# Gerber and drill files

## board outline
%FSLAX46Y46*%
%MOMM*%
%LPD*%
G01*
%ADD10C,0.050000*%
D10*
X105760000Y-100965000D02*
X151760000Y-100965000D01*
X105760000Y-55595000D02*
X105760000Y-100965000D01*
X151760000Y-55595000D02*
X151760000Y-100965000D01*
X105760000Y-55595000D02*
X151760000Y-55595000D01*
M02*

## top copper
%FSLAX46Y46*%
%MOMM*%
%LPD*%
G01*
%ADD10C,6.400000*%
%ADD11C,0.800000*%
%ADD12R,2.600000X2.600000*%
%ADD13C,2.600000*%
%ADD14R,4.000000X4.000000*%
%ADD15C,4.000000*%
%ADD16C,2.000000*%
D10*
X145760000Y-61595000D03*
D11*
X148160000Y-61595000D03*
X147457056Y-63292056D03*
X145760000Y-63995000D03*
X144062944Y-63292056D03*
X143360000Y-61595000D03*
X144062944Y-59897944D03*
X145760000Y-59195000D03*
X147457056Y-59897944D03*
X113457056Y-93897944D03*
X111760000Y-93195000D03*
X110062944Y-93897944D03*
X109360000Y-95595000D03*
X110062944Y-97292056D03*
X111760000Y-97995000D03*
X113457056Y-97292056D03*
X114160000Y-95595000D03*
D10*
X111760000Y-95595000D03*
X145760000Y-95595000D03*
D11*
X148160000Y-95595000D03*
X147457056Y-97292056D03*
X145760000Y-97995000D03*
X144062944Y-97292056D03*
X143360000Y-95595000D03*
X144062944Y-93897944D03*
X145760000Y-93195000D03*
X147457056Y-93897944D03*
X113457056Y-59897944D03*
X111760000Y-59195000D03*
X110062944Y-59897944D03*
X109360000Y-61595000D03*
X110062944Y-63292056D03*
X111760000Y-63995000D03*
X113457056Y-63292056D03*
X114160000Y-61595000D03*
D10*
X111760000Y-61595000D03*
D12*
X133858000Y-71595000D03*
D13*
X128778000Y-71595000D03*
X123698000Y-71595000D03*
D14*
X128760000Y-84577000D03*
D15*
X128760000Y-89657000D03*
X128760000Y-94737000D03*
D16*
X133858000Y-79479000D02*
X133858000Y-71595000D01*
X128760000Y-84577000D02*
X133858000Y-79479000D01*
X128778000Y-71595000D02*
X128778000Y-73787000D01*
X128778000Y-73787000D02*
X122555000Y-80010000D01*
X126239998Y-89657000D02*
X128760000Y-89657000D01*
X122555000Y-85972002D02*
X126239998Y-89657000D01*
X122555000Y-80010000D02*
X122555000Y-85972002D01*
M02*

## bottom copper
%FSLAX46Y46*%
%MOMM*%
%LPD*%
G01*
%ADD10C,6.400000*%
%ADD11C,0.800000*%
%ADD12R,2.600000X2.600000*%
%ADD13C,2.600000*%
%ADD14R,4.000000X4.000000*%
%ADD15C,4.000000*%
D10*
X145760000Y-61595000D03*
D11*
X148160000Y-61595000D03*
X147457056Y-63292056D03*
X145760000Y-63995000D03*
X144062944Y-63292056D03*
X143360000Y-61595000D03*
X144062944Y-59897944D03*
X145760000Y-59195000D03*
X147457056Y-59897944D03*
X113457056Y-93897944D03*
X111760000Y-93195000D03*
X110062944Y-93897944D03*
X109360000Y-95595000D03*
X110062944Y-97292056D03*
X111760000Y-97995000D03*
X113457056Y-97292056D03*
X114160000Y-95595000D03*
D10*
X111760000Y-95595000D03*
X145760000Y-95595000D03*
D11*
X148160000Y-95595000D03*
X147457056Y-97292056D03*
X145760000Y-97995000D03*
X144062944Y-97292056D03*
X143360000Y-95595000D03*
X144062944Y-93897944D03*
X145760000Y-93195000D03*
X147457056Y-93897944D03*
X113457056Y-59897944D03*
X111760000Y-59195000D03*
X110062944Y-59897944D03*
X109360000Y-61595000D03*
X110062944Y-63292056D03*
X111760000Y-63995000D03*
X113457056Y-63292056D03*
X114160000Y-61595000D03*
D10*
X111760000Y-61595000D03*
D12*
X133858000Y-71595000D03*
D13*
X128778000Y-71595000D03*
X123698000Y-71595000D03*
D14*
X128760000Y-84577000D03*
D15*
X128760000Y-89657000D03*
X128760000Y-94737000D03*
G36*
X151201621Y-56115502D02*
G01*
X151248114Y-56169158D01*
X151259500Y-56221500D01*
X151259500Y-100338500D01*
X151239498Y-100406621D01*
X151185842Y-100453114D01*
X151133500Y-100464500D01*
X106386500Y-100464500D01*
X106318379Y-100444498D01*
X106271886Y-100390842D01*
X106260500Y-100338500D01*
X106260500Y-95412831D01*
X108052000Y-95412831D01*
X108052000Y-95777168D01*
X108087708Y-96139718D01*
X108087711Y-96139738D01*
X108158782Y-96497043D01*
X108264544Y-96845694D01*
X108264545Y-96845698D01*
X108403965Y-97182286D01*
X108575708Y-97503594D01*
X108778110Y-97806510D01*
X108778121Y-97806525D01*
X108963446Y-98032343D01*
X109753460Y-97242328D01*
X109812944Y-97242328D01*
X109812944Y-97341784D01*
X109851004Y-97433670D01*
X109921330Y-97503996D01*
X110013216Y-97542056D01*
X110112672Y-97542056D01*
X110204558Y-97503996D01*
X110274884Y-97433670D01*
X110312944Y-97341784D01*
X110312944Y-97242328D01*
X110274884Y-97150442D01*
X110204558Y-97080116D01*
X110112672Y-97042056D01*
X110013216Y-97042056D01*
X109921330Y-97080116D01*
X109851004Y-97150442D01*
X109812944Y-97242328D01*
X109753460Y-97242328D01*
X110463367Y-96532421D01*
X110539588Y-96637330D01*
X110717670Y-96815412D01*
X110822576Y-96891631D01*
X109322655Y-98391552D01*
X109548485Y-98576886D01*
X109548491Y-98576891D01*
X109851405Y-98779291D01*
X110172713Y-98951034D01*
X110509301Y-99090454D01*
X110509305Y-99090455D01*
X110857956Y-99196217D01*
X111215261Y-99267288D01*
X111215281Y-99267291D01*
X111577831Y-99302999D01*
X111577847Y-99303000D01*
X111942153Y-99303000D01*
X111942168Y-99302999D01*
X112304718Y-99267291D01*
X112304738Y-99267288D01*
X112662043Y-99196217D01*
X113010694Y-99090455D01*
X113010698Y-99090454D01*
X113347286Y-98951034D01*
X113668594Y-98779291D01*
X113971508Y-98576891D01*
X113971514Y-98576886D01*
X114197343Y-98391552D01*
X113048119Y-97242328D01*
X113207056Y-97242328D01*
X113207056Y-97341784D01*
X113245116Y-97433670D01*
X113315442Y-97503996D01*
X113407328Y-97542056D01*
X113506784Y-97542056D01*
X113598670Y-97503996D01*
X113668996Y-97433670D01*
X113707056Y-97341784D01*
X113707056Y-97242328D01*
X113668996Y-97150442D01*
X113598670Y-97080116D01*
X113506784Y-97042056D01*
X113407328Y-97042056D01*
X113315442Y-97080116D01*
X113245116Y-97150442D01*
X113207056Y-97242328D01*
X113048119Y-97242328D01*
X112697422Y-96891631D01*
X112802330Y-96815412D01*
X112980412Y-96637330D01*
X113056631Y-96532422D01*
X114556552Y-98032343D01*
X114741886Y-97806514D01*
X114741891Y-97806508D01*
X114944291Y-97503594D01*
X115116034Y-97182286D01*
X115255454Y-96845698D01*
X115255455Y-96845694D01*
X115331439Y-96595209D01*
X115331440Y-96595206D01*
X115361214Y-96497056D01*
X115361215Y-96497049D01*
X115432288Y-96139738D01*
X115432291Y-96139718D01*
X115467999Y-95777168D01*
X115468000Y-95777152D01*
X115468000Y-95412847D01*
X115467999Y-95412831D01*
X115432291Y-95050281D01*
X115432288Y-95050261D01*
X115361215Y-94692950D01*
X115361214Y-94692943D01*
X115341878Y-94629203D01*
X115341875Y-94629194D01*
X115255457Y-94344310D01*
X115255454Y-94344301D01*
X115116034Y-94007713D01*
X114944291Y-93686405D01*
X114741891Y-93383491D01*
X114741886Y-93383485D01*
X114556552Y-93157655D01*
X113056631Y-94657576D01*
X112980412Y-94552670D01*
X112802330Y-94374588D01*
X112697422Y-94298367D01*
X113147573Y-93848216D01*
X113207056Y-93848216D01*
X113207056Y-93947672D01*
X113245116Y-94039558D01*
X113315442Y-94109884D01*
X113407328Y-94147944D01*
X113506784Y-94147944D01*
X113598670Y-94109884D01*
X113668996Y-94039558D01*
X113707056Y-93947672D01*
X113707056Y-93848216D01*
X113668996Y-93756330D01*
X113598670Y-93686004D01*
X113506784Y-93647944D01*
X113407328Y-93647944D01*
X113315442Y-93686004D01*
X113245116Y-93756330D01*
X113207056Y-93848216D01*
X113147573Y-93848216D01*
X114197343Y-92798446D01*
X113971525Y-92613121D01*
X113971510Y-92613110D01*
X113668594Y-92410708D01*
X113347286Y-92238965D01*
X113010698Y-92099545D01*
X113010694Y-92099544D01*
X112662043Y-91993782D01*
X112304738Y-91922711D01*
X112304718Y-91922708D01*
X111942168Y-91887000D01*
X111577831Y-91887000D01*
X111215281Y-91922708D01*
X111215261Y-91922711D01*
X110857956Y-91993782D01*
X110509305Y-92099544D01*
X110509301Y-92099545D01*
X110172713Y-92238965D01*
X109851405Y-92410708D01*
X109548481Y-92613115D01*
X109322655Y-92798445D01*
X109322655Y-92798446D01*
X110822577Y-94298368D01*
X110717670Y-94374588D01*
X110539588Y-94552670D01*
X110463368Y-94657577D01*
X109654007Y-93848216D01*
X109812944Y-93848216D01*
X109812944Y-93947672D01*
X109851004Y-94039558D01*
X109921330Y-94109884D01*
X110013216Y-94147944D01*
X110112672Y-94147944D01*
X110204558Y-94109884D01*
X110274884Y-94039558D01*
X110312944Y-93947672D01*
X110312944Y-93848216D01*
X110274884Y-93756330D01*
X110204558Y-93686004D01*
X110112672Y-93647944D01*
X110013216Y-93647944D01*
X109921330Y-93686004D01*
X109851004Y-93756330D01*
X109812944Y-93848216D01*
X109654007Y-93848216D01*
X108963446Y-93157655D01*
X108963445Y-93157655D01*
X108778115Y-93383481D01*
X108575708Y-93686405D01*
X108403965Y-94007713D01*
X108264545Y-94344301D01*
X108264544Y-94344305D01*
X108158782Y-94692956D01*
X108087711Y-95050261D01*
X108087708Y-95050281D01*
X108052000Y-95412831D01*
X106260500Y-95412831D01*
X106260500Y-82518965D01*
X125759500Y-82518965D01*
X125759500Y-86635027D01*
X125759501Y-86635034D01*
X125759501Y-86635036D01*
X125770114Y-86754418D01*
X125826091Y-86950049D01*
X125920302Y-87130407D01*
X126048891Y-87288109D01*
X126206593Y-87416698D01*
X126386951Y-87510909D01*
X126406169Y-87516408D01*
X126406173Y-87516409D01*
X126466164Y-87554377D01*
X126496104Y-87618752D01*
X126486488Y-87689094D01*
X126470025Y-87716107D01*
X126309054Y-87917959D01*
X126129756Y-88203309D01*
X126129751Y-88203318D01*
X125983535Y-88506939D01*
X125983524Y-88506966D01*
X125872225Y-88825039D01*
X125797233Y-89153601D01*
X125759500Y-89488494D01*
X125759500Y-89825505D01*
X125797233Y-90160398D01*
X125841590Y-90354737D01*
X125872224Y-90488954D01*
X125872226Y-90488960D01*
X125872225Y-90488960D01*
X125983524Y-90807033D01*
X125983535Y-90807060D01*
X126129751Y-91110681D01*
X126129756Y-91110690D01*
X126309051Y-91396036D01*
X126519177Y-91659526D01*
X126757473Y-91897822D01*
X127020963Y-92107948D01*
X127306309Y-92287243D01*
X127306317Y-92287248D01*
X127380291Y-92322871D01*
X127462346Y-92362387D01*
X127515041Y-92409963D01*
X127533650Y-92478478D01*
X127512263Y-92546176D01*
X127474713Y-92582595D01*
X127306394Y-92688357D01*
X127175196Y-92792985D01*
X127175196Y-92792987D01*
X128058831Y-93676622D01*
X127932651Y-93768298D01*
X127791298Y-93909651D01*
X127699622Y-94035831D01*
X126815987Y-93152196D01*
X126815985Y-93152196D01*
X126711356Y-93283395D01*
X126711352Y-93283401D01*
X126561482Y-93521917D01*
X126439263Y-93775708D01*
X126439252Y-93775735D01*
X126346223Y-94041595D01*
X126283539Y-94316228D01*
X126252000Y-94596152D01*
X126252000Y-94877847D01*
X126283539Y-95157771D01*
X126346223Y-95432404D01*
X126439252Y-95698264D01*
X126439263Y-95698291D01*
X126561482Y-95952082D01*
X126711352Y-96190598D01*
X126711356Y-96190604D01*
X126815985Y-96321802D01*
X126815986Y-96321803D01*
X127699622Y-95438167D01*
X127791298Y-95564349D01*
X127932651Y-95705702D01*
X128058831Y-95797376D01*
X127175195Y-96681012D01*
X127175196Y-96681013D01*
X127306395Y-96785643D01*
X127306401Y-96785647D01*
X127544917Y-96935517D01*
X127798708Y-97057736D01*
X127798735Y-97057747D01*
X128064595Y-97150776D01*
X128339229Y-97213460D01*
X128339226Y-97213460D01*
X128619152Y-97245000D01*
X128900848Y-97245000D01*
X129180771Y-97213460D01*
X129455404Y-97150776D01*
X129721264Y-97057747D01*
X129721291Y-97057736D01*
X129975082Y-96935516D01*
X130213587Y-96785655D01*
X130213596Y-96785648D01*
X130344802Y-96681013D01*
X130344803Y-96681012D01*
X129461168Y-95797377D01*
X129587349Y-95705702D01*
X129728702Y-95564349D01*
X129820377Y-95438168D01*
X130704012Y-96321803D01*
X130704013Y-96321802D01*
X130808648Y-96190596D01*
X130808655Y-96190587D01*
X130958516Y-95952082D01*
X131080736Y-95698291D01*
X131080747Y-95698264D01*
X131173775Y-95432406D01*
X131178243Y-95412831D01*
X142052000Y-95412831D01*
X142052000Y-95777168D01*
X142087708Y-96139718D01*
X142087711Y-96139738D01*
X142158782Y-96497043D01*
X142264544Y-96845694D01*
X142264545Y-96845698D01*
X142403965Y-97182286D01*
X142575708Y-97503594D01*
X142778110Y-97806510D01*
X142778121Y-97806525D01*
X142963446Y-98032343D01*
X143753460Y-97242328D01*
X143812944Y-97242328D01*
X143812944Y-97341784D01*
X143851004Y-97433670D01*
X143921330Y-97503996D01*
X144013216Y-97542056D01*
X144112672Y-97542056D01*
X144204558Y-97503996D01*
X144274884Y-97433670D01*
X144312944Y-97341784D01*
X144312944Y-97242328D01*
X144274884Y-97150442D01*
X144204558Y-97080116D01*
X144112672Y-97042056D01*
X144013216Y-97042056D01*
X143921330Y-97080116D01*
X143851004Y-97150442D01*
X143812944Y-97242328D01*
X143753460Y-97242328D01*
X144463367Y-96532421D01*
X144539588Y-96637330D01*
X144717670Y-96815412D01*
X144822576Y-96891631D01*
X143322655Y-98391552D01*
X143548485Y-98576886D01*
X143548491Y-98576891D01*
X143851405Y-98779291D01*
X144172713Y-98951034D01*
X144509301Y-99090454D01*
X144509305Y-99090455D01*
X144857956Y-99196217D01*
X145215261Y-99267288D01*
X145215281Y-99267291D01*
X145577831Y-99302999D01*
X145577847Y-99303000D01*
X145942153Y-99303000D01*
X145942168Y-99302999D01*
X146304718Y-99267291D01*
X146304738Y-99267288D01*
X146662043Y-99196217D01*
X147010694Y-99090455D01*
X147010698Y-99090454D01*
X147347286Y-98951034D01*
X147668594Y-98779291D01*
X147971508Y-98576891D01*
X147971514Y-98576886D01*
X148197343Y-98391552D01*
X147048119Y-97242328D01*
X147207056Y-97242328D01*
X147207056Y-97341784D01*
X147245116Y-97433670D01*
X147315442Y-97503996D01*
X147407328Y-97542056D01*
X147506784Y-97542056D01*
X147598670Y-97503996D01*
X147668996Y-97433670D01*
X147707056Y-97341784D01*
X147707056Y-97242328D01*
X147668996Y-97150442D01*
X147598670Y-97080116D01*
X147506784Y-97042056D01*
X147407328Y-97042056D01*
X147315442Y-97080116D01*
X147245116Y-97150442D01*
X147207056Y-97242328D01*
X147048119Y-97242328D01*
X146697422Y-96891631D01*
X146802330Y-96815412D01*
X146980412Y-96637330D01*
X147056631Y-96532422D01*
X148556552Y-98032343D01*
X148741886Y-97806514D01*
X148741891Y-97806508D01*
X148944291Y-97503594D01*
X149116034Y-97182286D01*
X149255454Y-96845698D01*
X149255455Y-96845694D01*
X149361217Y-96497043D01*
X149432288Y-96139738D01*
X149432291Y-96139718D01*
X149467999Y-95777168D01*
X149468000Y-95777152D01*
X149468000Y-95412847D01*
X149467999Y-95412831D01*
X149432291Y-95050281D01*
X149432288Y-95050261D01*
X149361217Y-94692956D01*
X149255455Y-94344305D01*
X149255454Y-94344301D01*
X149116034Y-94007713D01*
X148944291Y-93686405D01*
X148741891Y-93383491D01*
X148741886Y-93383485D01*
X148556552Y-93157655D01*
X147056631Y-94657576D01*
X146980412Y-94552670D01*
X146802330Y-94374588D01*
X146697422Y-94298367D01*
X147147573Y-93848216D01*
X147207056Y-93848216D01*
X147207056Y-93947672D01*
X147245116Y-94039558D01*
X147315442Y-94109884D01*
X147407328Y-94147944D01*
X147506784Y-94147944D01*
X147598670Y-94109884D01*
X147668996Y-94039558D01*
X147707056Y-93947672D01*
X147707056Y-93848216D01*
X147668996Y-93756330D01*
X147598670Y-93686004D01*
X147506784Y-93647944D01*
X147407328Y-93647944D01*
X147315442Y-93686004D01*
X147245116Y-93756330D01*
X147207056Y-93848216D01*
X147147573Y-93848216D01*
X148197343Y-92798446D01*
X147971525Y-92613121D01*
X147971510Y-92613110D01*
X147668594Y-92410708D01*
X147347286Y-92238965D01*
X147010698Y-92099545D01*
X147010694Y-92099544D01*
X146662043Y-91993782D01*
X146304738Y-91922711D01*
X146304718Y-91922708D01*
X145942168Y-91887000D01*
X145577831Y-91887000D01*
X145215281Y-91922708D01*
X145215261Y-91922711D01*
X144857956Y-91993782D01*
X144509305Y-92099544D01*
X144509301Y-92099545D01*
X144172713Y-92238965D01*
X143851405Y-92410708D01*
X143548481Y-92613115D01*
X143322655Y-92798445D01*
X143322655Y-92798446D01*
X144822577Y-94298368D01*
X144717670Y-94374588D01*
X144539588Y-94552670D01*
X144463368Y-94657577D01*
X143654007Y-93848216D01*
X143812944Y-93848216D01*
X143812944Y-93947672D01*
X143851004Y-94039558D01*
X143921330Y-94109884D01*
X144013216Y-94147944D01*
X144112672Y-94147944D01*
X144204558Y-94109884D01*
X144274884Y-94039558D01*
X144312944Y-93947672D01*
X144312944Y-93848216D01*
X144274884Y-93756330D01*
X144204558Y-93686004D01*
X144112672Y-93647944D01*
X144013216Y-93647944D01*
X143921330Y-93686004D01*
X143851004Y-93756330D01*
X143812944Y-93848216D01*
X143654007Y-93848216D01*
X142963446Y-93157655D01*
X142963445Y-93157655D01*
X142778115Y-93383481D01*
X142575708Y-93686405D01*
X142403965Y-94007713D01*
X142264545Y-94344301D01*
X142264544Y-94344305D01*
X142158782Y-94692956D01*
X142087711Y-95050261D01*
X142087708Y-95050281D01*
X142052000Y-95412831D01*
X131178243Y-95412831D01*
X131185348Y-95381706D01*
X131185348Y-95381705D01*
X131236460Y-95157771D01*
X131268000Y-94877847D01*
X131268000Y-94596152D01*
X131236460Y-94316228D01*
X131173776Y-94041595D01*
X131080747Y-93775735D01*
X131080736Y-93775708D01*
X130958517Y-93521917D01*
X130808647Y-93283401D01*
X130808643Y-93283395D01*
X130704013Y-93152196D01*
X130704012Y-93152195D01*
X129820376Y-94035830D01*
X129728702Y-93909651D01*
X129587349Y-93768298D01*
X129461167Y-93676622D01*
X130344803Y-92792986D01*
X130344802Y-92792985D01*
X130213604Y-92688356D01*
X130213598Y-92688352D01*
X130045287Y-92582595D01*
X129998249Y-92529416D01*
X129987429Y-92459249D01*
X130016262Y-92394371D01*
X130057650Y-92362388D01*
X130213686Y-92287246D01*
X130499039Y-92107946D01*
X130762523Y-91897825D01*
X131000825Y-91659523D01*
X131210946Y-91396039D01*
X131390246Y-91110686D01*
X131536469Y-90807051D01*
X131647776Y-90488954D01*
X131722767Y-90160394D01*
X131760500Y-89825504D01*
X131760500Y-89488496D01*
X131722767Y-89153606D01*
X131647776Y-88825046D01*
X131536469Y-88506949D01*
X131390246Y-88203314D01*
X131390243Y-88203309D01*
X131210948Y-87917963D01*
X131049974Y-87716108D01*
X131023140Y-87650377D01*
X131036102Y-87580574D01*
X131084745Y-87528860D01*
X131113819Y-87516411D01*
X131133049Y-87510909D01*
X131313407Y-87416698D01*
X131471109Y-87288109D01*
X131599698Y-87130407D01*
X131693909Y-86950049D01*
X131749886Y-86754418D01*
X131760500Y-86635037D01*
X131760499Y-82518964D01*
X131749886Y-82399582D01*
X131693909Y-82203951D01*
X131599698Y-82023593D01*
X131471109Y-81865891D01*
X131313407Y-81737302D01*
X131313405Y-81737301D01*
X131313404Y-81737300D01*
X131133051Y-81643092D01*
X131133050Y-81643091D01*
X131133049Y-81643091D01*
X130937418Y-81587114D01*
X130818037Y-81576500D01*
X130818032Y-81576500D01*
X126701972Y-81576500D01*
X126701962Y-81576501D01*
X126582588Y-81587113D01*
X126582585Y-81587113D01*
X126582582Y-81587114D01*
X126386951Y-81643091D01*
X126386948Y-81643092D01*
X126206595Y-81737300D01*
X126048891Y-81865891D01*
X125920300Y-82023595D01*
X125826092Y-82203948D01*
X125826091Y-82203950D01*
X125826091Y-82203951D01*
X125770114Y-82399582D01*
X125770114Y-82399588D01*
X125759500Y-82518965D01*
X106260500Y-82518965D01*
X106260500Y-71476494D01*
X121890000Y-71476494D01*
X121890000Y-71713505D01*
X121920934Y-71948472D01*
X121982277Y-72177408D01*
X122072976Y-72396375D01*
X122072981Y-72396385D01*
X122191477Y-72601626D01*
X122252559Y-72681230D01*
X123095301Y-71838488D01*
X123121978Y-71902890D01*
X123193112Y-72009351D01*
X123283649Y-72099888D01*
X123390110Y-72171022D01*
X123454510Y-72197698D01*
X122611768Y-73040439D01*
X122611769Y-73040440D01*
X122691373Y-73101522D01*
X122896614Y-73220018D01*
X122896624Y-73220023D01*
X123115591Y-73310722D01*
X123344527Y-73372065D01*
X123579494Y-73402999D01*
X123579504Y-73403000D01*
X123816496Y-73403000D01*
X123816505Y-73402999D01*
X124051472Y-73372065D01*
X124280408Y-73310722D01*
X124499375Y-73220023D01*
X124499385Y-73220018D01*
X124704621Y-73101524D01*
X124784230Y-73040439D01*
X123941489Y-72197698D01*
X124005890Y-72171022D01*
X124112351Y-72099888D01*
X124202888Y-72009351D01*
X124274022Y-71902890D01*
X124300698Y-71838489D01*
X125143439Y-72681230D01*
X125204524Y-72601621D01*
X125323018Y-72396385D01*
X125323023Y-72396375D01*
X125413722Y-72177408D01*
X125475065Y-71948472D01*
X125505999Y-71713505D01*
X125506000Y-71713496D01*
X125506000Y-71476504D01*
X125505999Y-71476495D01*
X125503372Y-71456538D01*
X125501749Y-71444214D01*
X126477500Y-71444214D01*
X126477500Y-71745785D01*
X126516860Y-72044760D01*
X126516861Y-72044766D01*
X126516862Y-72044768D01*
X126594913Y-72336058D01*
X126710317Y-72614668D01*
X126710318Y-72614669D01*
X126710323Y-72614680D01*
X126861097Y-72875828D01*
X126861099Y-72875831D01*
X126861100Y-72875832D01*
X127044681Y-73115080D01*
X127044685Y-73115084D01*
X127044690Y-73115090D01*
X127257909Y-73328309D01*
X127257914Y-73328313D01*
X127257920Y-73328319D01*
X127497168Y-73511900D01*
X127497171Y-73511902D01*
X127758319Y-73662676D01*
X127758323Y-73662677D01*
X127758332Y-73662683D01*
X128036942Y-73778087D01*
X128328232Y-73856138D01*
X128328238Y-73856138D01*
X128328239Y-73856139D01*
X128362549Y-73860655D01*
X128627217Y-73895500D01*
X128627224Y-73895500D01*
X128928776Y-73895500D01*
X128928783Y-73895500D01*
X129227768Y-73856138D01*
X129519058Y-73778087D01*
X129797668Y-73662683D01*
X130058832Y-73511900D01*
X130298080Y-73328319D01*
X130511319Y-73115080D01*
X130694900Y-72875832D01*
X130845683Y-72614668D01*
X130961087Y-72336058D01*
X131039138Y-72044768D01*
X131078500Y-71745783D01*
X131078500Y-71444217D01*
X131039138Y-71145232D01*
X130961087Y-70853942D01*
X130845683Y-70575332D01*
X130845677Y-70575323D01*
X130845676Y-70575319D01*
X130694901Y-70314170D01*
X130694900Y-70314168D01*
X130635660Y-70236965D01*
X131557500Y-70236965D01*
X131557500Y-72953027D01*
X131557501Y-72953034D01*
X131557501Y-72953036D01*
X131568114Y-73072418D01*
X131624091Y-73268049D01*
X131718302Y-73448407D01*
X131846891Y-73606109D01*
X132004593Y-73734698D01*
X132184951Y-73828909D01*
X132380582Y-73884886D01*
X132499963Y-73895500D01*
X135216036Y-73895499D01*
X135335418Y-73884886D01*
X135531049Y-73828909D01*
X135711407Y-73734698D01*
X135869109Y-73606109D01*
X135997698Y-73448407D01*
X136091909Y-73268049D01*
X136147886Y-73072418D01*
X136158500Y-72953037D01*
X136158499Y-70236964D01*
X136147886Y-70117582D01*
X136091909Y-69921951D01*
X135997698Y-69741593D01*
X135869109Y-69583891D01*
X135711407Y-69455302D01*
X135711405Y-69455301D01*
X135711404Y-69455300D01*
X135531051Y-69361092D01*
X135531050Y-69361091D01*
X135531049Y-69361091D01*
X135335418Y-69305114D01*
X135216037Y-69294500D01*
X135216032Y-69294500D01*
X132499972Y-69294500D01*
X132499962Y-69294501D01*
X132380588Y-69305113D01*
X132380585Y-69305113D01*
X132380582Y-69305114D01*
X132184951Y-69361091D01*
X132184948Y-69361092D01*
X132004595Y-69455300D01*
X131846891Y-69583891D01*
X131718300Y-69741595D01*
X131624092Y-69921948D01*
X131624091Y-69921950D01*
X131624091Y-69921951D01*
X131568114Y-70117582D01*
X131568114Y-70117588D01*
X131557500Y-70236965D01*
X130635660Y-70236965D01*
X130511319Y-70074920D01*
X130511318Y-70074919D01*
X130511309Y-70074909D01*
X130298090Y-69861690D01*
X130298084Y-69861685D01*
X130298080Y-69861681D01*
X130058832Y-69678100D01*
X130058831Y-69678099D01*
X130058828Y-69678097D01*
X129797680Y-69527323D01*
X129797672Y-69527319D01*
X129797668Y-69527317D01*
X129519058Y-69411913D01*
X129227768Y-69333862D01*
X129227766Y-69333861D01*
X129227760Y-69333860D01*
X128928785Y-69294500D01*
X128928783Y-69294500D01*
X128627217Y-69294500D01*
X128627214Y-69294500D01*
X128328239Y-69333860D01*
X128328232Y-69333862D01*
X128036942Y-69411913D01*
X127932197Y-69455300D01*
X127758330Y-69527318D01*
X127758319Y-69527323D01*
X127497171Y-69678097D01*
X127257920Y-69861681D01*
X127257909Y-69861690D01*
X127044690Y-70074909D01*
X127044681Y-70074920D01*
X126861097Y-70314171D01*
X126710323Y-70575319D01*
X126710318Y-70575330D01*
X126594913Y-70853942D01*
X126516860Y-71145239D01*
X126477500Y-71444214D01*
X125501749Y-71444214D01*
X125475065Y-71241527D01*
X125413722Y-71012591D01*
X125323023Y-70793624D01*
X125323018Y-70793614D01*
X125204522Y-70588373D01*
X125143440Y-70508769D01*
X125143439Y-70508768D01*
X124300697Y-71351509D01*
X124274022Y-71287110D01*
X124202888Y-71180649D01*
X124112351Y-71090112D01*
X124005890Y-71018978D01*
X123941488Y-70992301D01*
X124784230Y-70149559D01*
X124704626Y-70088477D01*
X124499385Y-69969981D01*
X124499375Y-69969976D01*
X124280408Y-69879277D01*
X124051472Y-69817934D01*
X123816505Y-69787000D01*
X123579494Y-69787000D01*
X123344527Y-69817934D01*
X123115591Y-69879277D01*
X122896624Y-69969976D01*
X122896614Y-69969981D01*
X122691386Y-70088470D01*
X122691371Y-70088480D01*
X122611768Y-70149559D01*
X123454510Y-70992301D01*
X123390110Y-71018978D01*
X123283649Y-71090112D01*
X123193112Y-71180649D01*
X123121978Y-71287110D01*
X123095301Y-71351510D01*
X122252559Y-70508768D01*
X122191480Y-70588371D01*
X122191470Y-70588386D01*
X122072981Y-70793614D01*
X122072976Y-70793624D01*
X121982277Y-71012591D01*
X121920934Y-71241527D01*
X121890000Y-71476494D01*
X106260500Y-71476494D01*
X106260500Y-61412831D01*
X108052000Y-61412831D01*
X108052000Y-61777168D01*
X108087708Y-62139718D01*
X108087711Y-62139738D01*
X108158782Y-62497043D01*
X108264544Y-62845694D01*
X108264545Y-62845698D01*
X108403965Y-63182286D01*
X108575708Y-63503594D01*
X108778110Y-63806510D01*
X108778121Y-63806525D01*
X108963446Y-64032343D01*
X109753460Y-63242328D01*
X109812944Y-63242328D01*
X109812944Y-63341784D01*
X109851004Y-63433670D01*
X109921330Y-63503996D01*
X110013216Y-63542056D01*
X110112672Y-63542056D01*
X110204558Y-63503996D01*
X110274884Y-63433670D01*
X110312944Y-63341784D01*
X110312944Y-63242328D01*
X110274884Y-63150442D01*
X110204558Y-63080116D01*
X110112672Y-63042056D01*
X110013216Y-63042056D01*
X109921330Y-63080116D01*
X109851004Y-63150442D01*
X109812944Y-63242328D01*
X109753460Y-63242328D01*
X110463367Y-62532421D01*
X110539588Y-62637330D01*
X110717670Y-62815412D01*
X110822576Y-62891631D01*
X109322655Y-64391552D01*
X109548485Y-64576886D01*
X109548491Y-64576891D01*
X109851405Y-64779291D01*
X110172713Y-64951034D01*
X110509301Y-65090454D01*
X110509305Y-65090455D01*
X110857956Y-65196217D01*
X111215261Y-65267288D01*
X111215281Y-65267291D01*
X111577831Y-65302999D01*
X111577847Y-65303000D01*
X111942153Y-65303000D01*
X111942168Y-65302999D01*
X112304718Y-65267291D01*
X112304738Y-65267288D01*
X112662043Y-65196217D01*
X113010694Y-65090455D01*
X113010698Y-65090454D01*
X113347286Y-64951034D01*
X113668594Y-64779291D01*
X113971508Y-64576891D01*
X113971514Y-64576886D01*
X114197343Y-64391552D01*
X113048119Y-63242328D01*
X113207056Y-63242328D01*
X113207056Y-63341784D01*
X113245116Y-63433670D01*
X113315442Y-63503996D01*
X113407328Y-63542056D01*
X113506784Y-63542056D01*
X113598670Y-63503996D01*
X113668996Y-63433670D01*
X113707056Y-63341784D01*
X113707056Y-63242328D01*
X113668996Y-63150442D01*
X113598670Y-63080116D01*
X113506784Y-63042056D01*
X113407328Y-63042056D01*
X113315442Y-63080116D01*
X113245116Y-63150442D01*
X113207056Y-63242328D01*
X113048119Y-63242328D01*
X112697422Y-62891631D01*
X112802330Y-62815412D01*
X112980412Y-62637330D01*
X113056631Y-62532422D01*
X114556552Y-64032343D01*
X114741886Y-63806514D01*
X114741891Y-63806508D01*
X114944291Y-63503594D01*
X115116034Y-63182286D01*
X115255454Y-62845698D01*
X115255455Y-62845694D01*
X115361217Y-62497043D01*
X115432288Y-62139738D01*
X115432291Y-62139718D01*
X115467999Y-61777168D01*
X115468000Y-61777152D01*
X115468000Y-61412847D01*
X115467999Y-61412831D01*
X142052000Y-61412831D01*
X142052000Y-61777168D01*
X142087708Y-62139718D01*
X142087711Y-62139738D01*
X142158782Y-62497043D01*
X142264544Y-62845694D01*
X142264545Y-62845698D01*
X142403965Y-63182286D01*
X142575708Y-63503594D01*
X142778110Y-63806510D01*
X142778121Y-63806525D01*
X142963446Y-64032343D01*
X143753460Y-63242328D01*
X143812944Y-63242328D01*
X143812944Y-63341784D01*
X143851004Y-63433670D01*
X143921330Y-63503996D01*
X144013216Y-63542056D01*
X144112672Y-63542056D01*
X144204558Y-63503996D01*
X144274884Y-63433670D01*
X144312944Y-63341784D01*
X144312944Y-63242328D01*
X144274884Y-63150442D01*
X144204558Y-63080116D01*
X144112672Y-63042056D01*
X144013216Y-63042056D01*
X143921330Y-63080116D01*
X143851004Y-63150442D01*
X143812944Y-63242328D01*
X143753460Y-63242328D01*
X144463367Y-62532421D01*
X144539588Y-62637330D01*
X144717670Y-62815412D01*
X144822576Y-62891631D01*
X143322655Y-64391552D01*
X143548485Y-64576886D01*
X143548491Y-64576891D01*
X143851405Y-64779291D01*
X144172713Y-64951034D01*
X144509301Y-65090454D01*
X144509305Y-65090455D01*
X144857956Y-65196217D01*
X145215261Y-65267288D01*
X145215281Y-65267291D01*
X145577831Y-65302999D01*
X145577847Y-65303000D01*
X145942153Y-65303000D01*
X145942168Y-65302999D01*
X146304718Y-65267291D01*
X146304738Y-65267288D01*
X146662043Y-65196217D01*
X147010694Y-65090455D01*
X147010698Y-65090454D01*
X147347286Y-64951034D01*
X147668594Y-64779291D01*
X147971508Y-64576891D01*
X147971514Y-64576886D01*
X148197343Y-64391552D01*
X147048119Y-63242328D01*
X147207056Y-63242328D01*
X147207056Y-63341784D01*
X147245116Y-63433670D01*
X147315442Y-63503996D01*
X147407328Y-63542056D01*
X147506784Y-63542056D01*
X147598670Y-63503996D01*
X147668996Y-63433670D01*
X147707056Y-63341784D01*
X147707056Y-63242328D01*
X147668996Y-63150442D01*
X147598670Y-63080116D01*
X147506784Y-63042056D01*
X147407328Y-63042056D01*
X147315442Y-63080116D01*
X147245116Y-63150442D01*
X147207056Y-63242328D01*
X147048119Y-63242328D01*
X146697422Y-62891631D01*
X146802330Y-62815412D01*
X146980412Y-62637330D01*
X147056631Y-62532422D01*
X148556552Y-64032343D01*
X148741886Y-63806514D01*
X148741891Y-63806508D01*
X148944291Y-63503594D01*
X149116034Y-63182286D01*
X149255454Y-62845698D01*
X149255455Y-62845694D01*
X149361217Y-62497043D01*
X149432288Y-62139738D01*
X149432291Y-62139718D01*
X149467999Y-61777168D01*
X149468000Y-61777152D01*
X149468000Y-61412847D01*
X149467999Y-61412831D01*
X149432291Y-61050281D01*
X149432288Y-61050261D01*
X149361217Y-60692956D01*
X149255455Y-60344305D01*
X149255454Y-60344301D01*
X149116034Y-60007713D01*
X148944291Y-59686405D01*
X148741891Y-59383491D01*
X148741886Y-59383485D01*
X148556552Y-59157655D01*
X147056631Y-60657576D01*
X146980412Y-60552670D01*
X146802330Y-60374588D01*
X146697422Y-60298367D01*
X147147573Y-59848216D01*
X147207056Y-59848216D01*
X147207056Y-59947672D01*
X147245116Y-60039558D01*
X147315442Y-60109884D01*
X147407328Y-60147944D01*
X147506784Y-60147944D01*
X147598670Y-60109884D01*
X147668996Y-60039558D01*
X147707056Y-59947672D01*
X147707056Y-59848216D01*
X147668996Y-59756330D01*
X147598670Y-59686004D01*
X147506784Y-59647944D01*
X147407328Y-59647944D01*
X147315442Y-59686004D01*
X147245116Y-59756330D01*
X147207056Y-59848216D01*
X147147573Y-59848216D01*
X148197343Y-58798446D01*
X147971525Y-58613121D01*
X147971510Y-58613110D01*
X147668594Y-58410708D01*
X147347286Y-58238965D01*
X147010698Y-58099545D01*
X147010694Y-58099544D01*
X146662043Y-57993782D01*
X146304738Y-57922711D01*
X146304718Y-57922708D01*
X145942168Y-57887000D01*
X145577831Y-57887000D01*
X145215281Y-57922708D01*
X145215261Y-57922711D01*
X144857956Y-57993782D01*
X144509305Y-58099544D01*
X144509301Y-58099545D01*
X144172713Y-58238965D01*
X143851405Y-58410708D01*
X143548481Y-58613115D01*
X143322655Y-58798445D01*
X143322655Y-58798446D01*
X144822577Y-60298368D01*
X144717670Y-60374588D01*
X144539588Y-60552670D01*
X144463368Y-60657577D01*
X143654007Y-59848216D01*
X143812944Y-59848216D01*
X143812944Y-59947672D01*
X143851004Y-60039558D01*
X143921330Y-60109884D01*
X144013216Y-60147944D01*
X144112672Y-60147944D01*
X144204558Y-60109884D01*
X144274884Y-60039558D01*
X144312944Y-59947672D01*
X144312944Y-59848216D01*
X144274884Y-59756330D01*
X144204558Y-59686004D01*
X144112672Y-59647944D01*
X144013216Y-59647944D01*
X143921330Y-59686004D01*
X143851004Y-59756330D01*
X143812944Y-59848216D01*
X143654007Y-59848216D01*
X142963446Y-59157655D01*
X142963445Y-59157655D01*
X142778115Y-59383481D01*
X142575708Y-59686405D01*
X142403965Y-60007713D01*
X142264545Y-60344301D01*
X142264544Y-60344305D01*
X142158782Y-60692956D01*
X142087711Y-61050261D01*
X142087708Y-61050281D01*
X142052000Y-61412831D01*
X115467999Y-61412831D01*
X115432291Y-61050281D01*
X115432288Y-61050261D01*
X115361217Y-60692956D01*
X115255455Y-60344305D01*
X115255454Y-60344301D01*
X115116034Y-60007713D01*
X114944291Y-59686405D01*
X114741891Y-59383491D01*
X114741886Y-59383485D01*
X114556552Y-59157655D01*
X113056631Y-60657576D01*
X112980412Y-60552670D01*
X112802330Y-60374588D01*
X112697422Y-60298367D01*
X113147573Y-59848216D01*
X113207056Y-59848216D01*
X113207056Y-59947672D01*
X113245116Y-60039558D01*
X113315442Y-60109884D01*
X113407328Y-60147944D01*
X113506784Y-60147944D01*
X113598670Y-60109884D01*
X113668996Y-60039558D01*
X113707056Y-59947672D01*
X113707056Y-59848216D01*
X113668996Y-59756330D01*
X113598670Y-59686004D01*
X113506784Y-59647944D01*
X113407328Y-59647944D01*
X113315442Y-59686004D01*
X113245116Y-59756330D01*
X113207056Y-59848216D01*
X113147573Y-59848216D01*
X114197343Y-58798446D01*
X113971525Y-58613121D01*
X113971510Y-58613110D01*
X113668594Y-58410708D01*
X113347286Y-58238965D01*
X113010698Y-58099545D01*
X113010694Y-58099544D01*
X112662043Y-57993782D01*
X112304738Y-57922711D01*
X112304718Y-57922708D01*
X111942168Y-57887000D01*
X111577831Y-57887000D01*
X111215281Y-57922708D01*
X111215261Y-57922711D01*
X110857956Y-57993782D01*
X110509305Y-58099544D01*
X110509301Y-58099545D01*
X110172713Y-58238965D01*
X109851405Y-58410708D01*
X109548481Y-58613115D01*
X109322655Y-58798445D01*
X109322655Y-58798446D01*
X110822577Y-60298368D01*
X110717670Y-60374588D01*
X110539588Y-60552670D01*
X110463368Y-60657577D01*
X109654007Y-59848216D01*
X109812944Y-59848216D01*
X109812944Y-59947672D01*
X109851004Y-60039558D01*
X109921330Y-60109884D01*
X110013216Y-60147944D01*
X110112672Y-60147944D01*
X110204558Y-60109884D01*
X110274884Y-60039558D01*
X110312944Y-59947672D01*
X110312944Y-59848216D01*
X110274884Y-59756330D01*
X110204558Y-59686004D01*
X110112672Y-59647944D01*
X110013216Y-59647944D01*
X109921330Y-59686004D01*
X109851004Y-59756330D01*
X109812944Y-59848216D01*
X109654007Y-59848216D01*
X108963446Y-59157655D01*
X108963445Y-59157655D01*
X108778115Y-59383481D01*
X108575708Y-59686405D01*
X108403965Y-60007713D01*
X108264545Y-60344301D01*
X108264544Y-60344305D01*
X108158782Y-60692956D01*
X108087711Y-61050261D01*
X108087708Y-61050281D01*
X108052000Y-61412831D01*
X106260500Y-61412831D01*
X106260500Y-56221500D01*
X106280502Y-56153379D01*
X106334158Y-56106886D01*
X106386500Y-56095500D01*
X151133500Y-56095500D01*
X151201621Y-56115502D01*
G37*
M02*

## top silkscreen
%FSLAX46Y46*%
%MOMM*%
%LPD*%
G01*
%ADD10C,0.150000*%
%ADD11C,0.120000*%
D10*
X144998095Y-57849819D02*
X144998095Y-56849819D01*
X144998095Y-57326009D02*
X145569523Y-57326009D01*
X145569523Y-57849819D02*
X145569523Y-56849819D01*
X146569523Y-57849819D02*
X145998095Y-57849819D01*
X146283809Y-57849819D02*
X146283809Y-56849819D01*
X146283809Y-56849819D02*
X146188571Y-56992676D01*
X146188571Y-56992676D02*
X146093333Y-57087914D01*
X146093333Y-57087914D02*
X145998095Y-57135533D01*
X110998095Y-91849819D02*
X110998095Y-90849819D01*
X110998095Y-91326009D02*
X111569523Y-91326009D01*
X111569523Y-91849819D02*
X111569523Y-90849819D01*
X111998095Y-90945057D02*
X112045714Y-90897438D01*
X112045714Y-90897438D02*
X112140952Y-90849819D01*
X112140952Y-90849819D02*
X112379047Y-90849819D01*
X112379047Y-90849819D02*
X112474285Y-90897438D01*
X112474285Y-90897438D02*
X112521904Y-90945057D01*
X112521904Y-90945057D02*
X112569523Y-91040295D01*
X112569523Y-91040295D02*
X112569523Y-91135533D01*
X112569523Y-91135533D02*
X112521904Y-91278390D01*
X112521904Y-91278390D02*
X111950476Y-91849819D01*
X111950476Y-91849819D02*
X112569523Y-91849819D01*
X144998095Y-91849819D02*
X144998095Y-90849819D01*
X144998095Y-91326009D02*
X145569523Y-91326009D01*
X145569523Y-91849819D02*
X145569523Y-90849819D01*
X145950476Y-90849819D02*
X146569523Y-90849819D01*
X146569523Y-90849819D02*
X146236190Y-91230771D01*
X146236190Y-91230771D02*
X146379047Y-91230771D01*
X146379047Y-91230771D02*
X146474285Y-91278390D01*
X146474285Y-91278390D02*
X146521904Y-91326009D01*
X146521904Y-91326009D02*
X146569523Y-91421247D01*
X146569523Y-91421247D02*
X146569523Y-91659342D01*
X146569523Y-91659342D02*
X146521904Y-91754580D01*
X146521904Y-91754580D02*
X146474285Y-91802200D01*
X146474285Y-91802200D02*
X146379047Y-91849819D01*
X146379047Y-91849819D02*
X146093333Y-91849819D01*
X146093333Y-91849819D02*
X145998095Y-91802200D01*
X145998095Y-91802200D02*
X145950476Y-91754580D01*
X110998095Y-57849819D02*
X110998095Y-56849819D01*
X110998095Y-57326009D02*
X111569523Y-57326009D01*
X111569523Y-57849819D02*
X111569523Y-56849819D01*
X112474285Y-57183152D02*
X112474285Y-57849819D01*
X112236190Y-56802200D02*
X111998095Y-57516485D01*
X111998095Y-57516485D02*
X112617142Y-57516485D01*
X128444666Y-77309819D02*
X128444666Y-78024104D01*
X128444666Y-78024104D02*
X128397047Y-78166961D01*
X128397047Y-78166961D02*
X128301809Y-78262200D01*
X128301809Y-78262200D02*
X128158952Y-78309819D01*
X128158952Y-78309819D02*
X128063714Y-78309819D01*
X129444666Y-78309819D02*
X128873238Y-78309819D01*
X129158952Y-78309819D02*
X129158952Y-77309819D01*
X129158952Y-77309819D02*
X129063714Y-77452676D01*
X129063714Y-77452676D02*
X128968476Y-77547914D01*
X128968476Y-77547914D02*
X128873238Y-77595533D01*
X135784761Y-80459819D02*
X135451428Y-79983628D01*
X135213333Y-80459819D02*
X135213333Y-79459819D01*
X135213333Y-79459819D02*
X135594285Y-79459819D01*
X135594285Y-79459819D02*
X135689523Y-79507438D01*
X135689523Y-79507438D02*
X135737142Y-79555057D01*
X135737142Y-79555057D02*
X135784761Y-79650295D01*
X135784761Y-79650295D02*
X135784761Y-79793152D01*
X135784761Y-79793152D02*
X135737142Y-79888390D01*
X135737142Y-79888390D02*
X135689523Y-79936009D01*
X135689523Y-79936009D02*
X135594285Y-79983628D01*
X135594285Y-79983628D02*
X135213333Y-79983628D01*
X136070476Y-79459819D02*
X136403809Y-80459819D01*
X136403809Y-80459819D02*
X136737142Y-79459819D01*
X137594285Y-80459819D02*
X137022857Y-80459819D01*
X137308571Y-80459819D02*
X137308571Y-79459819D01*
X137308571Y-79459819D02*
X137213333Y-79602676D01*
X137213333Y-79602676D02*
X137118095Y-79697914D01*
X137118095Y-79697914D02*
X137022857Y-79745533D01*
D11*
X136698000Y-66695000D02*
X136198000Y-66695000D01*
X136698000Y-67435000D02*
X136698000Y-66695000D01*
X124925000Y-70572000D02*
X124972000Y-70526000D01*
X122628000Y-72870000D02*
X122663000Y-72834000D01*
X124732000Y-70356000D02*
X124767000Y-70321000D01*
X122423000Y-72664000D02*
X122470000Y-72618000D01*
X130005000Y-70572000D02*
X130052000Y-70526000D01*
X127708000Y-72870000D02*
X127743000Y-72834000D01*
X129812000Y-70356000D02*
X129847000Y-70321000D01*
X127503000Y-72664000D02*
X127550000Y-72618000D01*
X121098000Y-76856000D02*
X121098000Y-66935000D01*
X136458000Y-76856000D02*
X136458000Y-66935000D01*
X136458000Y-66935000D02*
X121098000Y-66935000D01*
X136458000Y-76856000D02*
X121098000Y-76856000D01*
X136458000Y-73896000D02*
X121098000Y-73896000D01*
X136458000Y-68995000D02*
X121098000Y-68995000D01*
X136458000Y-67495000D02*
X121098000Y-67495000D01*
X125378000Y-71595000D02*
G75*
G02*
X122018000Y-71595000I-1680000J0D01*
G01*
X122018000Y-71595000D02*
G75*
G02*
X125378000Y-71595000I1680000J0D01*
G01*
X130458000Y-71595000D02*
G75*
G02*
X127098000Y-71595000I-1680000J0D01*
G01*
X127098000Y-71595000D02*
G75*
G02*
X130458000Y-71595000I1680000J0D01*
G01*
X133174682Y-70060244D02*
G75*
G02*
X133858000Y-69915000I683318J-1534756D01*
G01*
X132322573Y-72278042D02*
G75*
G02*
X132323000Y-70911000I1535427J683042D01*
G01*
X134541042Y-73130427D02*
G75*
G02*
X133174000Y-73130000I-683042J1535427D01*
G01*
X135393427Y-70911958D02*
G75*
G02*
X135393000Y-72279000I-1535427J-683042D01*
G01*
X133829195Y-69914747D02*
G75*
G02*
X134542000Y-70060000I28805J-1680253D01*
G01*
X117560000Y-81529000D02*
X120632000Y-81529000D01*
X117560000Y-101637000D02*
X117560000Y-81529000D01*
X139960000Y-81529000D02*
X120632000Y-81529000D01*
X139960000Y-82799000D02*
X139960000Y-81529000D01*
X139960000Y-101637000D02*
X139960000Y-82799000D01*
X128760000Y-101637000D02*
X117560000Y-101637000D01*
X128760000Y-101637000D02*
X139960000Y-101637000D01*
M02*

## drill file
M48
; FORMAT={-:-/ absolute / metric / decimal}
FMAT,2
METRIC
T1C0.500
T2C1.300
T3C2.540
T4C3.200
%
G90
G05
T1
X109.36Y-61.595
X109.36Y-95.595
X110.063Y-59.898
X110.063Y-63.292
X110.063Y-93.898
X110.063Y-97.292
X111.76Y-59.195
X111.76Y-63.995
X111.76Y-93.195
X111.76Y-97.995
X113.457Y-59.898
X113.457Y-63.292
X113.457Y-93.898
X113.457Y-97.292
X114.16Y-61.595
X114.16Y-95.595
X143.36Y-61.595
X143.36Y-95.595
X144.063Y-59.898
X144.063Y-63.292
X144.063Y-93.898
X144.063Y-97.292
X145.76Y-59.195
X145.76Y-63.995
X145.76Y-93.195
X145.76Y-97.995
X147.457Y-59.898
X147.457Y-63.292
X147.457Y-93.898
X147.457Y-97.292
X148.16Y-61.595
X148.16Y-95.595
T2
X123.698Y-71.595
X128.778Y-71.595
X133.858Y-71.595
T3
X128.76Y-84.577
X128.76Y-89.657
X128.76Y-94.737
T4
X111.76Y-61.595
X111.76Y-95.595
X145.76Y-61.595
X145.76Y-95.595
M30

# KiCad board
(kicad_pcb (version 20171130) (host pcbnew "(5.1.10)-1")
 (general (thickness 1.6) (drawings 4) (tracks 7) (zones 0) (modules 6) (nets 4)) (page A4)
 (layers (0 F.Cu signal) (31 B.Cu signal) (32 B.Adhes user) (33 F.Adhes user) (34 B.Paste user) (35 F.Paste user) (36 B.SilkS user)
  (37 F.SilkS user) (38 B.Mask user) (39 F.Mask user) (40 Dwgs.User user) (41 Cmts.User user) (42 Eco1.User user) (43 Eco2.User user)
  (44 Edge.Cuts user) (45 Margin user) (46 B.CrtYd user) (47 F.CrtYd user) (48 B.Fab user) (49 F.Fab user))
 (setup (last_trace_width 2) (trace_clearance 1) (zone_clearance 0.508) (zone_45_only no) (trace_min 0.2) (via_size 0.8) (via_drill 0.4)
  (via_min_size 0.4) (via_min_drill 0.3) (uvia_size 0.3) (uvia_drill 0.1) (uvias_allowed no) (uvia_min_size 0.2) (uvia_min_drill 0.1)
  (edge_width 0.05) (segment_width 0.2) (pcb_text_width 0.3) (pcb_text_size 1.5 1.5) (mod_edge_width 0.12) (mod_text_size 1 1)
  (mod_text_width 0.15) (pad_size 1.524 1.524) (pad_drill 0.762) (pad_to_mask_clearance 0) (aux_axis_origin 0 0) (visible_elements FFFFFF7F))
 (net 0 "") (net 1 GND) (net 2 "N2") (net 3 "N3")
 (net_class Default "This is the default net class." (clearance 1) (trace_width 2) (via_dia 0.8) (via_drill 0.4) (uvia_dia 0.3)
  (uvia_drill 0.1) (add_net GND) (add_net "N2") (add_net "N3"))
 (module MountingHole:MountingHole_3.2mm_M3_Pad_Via (layer F.Cu) (at 145.76 61.595)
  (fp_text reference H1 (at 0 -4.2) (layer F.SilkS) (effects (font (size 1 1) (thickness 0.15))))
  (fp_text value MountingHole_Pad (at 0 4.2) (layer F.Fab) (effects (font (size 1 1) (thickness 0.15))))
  (pad 1 thru_hole circle (at 0 0) (size 6.4 6.4) (drill 3.2) (layers *.Cu *.Mask) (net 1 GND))
  (pad 1 thru_hole circle (at 2.4 0) (size 0.8 0.8) (drill 0.5) (layers *.Cu *.Mask) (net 1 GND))
  (pad 1 thru_hole circle (at 1.697056 1.697056) (size 0.8 0.8) (drill 0.5) (layers *.Cu *.Mask) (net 1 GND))
  (pad 1 thru_hole circle (at 0 2.4) (size 0.8 0.8) (drill 0.5) (layers *.Cu *.Mask) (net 1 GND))
  (pad 1 thru_hole circle (at -1.697056 1.697056) (size 0.8 0.8) (drill 0.5) (layers *.Cu *.Mask) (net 1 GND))
  (pad 1 thru_hole circle (at -2.4 0) (size 0.8 0.8) (drill 0.5) (layers *.Cu *.Mask) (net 1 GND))
  (pad 1 thru_hole circle (at -1.697056 -1.697056) (size 0.8 0.8) (drill 0.5) (layers *.Cu *.Mask) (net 1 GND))
  (pad 1 thru_hole circle (at 0 -2.4) (size 0.8 0.8) (drill 0.5) (layers *.Cu *.Mask) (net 1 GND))
  (pad 1 thru_hole circle (at 1.697056 -1.697056) (size 0.8 0.8) (drill 0.5) (layers *.Cu *.Mask) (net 1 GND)))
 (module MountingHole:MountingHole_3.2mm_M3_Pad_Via (layer F.Cu) (at 111.76 95.595)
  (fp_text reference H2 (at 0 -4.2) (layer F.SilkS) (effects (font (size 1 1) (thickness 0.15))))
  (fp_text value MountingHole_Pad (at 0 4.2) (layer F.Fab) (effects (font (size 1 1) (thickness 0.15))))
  (pad 1 thru_hole circle (at 1.697056 -1.697056) (size 0.8 0.8) (drill 0.5) (layers *.Cu *.Mask) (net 1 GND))
  (pad 1 thru_hole circle (at 0 -2.4) (size 0.8 0.8) (drill 0.5) (layers *.Cu *.Mask) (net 1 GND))
  (pad 1 thru_hole circle (at -1.697056 -1.697056) (size 0.8 0.8) (drill 0.5) (layers *.Cu *.Mask) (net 1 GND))
  (pad 1 thru_hole circle (at -2.4 0) (size 0.8 0.8) (drill 0.5) (layers *.Cu *.Mask) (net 1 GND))
  (pad 1 thru_hole circle (at -1.697056 1.697056) (size 0.8 0.8) (drill 0.5) (layers *.Cu *.Mask) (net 1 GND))
  (pad 1 thru_hole circle (at 0 2.4) (size 0.8 0.8) (drill 0.5) (layers *.Cu *.Mask) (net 1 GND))
  (pad 1 thru_hole circle (at 1.697056 1.697056) (size 0.8 0.8) (drill 0.5) (layers *.Cu *.Mask) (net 1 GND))
  (pad 1 thru_hole circle (at 2.4 0) (size 0.8 0.8) (drill 0.5) (layers *.Cu *.Mask) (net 1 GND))
  (pad 1 thru_hole circle (at 0 0) (size 6.4 6.4) (drill 3.2) (layers *.Cu *.Mask) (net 1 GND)))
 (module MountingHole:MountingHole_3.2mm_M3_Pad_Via (layer F.Cu) (at 145.76 95.595)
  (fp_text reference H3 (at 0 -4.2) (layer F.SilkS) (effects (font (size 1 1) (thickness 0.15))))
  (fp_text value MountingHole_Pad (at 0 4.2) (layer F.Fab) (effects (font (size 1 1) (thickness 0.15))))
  (pad 1 thru_hole circle (at 0 0) (size 6.4 6.4) (drill 3.2) (layers *.Cu *.Mask) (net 1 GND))
  (pad 1 thru_hole circle (at 2.4 0) (size 0.8 0.8) (drill 0.5) (layers *.Cu *.Mask) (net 1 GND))
  (pad 1 thru_hole circle (at 1.697056 1.697056) (size 0.8 0.8) (drill 0.5) (layers *.Cu *.Mask) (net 1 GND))
  (pad 1 thru_hole circle (at 0 2.4) (size 0.8 0.8) (drill 0.5) (layers *.Cu *.Mask) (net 1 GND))
  (pad 1 thru_hole circle (at -1.697056 1.697056) (size 0.8 0.8) (drill 0.5) (layers *.Cu *.Mask) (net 1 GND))
  (pad 1 thru_hole circle (at -2.4 0) (size 0.8 0.8) (drill 0.5) (layers *.Cu *.Mask) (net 1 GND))
  (pad 1 thru_hole circle (at -1.697056 -1.697056) (size 0.8 0.8) (drill 0.5) (layers *.Cu *.Mask) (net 1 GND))
  (pad 1 thru_hole circle (at 0 -2.4) (size 0.8 0.8) (drill 0.5) (layers *.Cu *.Mask) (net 1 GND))
  (pad 1 thru_hole circle (at 1.697056 -1.697056) (size 0.8 0.8) (drill 0.5) (layers *.Cu *.Mask) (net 1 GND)))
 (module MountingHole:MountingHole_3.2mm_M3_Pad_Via (layer F.Cu) (at 111.76 61.595)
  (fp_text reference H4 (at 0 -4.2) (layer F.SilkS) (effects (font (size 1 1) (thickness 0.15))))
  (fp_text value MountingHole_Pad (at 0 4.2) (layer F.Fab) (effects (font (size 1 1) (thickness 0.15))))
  (pad 1 thru_hole circle (at 1.697056 -1.697056) (size 0.8 0.8) (drill 0.5) (layers *.Cu *.Mask) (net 1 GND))
  (pad 1 thru_hole circle (at 0 -2.4) (size 0.8 0.8) (drill 0.5) (layers *.Cu *.Mask) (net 1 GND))
  (pad 1 thru_hole circle (at -1.697056 -1.697056) (size 0.8 0.8) (drill 0.5) (layers *.Cu *.Mask) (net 1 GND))
  (pad 1 thru_hole circle (at -2.4 0) (size 0.8 0.8) (drill 0.5) (layers *.Cu *.Mask) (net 1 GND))
  (pad 1 thru_hole circle (at -1.697056 1.697056) (size 0.8 0.8) (drill 0.5) (layers *.Cu *.Mask) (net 1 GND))
  (pad 1 thru_hole circle (at 0 2.4) (size 0.8 0.8) (drill 0.5) (layers *.Cu *.Mask) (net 1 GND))
  (pad 1 thru_hole circle (at 1.697056 1.697056) (size 0.8 0.8) (drill 0.5) (layers *.Cu *.Mask) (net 1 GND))
  (pad 1 thru_hole circle (at 2.4 0) (size 0.8 0.8) (drill 0.5) (layers *.Cu *.Mask) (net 1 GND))
  (pad 1 thru_hole circle (at 0 0) (size 6.4 6.4) (drill 3.2) (layers *.Cu *.Mask) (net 1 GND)))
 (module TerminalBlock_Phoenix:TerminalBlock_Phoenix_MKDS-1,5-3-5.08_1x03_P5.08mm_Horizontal (layer F.Cu) (at 133.858 71.595 180)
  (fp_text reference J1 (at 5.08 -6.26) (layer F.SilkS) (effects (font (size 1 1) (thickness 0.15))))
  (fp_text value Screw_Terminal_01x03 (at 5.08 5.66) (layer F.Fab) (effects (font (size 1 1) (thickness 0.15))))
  (fp_line (start -2.84 4.9) (end -2.34 4.9) (layer F.SilkS) (width 0.12))
  (fp_line (start -2.84 4.16) (end -2.84 4.9) (layer F.SilkS) (width 0.12))
  (fp_line (start 8.933 1.023) (end 8.886 1.069) (layer F.SilkS) (width 0.12))
  (fp_line (start 11.23 -1.275) (end 11.195 -1.239) (layer F.SilkS) (width 0.12))
  (fp_line (start 9.126 1.239) (end 9.091 1.274) (layer F.SilkS) (width 0.12))
  (fp_line (start 11.435 -1.069) (end 11.388 -1.023) (layer F.SilkS) (width 0.12))
  (fp_line (start 3.853 1.023) (end 3.806 1.069) (layer F.SilkS) (width 0.12))
  (fp_line (start 6.15 -1.275) (end 6.115 -1.239) (layer F.SilkS) (width 0.12))
  (fp_line (start 4.046 1.239) (end 4.011 1.274) (layer F.SilkS) (width 0.12))
  (fp_line (start 6.355 -1.069) (end 6.308 -1.023) (layer F.SilkS) (width 0.12))
  (fp_line (start 12.76 -5.261) (end 12.76 4.66) (layer F.SilkS) (width 0.12))
  (fp_line (start -2.6 -5.261) (end -2.6 4.66) (layer F.SilkS) (width 0.12))
  (fp_line (start -2.6 4.66) (end 12.76 4.66) (layer F.SilkS) (width 0.12))
  (fp_line (start -2.6 -5.261) (end 12.76 -5.261) (layer F.SilkS) (width 0.12))
  (fp_line (start -2.6 -2.301) (end 12.76 -2.301) (layer F.SilkS) (width 0.12))
  (fp_line (start -2.6 2.6) (end 12.76 2.6) (layer F.SilkS) (width 0.12))
  (fp_line (start -2.6 4.1) (end 12.76 4.1) (layer F.SilkS) (width 0.12))
  (fp_circle (center 10.16 0) (end 11.84 0) (layer F.SilkS) (width 0.12))
  (fp_circle (center 5.08 0) (end 6.76 0) (layer F.SilkS) (width 0.12))
  (fp_arc (start 0 0) (end 0 1.68) (angle -24) (layer F.SilkS) (width 0.12))
  (fp_arc (start 0 0) (end 1.535 0.684) (angle -48) (layer F.SilkS) (width 0.12))
  (fp_arc (start 0 0) (end 0.684 -1.535) (angle -48) (layer F.SilkS) (width 0.12))
  (fp_arc (start 0 0) (end -1.535 -0.684) (angle -48) (layer F.SilkS) (width 0.12))
  (fp_arc (start 0 0) (end -0.684 1.535) (angle -25) (layer F.SilkS) (width 0.12))
  (pad 1 thru_hole rect (at 0 0 180) (size 2.6 2.6) (drill 1.3) (layers *.Cu *.Mask) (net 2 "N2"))
  (pad 2 thru_hole circle (at 5.08 0 180) (size 2.6 2.6) (drill 1.3) (layers *.Cu *.Mask) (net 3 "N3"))
  (pad 3 thru_hole circle (at 10.16 0 180) (size 2.6 2.6) (drill 1.3) (layers *.Cu *.Mask) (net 1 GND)))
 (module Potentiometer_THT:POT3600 (layer F.Cu) (at 128.76 101.595)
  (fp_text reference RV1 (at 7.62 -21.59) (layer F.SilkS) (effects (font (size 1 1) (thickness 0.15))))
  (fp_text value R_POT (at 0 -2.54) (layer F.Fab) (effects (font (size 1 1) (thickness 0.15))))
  (fp_line (start -11.2 -20.066) (end -8.128 -20.066) (layer F.SilkS) (width 0.12))
  (fp_line (start -11.2 0.042) (end -11.2 -20.066) (layer F.SilkS) (width 0.12))
  (fp_line (start 11.2 -20.066) (end -8.128 -20.066) (layer F.SilkS) (width 0.12))
  (fp_line (start 11.2 -18.796) (end 11.2 -20.066) (layer F.SilkS) (width 0.12))
  (fp_line (start 11.2 0.042) (end 11.2 -18.796) (layer F.SilkS) (width 0.12))
  (fp_line (start 0 0.042) (end -11.2 0.042) (layer F.SilkS) (width 0.12))
  (fp_line (start 0 0.042) (end 11.2 0.042) (layer F.SilkS) (width 0.12))
  (pad 2 thru_hole rect (at 0 -17.018) (size 4 4) (drill 2.54) (layers *.Cu *.Mask) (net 2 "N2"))
  (pad 1 thru_hole circle (at 0 -11.938) (size 4 4) (drill 2.54) (layers *.Cu *.Mask) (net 3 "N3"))
  (pad 3 thru_hole circle (at 0 -6.858) (size 4 4) (drill 2.54) (layers *.Cu *.Mask) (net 1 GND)))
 (gr_line (start 105.76 100.965) (end 151.76 100.965) (layer Edge.Cuts) (width 0.05))
 (gr_line (start 105.76 55.595) (end 105.76 100.965) (layer Edge.Cuts) (width 0.05))
 (gr_line (start 151.76 55.595) (end 151.76 100.965) (layer Edge.Cuts) (width 0.05))
 (gr_line (start 105.76 55.595) (end 151.76 55.595) (layer Edge.Cuts) (width 0.05))
 (segment (start 133.858 79.479) (end 133.858 71.595) (width 2) (layer F.Cu) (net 2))
 (segment (start 128.76 84.577) (end 133.858 79.479) (width 2) (layer F.Cu) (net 2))
 (segment (start 128.778 71.595) (end 128.778 73.787) (width 2) (layer F.Cu) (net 3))
 (segment (start 128.778 73.787) (end 122.555 80.01) (width 2) (layer F.Cu) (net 3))
 (segment (start 126.239998 89.657) (end 128.76 89.657) (width 2) (layer F.Cu) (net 3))
 (segment (start 122.555 85.972002) (end 126.239998 89.657) (width 2) (layer F.Cu) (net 3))
 (segment (start 122.555 80.01) (end 122.555 85.972002) (width 2) (layer F.Cu) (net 3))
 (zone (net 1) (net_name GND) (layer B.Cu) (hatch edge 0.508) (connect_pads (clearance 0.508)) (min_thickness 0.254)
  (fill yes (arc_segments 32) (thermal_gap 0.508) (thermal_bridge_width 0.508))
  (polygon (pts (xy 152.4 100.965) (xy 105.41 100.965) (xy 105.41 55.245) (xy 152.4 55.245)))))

